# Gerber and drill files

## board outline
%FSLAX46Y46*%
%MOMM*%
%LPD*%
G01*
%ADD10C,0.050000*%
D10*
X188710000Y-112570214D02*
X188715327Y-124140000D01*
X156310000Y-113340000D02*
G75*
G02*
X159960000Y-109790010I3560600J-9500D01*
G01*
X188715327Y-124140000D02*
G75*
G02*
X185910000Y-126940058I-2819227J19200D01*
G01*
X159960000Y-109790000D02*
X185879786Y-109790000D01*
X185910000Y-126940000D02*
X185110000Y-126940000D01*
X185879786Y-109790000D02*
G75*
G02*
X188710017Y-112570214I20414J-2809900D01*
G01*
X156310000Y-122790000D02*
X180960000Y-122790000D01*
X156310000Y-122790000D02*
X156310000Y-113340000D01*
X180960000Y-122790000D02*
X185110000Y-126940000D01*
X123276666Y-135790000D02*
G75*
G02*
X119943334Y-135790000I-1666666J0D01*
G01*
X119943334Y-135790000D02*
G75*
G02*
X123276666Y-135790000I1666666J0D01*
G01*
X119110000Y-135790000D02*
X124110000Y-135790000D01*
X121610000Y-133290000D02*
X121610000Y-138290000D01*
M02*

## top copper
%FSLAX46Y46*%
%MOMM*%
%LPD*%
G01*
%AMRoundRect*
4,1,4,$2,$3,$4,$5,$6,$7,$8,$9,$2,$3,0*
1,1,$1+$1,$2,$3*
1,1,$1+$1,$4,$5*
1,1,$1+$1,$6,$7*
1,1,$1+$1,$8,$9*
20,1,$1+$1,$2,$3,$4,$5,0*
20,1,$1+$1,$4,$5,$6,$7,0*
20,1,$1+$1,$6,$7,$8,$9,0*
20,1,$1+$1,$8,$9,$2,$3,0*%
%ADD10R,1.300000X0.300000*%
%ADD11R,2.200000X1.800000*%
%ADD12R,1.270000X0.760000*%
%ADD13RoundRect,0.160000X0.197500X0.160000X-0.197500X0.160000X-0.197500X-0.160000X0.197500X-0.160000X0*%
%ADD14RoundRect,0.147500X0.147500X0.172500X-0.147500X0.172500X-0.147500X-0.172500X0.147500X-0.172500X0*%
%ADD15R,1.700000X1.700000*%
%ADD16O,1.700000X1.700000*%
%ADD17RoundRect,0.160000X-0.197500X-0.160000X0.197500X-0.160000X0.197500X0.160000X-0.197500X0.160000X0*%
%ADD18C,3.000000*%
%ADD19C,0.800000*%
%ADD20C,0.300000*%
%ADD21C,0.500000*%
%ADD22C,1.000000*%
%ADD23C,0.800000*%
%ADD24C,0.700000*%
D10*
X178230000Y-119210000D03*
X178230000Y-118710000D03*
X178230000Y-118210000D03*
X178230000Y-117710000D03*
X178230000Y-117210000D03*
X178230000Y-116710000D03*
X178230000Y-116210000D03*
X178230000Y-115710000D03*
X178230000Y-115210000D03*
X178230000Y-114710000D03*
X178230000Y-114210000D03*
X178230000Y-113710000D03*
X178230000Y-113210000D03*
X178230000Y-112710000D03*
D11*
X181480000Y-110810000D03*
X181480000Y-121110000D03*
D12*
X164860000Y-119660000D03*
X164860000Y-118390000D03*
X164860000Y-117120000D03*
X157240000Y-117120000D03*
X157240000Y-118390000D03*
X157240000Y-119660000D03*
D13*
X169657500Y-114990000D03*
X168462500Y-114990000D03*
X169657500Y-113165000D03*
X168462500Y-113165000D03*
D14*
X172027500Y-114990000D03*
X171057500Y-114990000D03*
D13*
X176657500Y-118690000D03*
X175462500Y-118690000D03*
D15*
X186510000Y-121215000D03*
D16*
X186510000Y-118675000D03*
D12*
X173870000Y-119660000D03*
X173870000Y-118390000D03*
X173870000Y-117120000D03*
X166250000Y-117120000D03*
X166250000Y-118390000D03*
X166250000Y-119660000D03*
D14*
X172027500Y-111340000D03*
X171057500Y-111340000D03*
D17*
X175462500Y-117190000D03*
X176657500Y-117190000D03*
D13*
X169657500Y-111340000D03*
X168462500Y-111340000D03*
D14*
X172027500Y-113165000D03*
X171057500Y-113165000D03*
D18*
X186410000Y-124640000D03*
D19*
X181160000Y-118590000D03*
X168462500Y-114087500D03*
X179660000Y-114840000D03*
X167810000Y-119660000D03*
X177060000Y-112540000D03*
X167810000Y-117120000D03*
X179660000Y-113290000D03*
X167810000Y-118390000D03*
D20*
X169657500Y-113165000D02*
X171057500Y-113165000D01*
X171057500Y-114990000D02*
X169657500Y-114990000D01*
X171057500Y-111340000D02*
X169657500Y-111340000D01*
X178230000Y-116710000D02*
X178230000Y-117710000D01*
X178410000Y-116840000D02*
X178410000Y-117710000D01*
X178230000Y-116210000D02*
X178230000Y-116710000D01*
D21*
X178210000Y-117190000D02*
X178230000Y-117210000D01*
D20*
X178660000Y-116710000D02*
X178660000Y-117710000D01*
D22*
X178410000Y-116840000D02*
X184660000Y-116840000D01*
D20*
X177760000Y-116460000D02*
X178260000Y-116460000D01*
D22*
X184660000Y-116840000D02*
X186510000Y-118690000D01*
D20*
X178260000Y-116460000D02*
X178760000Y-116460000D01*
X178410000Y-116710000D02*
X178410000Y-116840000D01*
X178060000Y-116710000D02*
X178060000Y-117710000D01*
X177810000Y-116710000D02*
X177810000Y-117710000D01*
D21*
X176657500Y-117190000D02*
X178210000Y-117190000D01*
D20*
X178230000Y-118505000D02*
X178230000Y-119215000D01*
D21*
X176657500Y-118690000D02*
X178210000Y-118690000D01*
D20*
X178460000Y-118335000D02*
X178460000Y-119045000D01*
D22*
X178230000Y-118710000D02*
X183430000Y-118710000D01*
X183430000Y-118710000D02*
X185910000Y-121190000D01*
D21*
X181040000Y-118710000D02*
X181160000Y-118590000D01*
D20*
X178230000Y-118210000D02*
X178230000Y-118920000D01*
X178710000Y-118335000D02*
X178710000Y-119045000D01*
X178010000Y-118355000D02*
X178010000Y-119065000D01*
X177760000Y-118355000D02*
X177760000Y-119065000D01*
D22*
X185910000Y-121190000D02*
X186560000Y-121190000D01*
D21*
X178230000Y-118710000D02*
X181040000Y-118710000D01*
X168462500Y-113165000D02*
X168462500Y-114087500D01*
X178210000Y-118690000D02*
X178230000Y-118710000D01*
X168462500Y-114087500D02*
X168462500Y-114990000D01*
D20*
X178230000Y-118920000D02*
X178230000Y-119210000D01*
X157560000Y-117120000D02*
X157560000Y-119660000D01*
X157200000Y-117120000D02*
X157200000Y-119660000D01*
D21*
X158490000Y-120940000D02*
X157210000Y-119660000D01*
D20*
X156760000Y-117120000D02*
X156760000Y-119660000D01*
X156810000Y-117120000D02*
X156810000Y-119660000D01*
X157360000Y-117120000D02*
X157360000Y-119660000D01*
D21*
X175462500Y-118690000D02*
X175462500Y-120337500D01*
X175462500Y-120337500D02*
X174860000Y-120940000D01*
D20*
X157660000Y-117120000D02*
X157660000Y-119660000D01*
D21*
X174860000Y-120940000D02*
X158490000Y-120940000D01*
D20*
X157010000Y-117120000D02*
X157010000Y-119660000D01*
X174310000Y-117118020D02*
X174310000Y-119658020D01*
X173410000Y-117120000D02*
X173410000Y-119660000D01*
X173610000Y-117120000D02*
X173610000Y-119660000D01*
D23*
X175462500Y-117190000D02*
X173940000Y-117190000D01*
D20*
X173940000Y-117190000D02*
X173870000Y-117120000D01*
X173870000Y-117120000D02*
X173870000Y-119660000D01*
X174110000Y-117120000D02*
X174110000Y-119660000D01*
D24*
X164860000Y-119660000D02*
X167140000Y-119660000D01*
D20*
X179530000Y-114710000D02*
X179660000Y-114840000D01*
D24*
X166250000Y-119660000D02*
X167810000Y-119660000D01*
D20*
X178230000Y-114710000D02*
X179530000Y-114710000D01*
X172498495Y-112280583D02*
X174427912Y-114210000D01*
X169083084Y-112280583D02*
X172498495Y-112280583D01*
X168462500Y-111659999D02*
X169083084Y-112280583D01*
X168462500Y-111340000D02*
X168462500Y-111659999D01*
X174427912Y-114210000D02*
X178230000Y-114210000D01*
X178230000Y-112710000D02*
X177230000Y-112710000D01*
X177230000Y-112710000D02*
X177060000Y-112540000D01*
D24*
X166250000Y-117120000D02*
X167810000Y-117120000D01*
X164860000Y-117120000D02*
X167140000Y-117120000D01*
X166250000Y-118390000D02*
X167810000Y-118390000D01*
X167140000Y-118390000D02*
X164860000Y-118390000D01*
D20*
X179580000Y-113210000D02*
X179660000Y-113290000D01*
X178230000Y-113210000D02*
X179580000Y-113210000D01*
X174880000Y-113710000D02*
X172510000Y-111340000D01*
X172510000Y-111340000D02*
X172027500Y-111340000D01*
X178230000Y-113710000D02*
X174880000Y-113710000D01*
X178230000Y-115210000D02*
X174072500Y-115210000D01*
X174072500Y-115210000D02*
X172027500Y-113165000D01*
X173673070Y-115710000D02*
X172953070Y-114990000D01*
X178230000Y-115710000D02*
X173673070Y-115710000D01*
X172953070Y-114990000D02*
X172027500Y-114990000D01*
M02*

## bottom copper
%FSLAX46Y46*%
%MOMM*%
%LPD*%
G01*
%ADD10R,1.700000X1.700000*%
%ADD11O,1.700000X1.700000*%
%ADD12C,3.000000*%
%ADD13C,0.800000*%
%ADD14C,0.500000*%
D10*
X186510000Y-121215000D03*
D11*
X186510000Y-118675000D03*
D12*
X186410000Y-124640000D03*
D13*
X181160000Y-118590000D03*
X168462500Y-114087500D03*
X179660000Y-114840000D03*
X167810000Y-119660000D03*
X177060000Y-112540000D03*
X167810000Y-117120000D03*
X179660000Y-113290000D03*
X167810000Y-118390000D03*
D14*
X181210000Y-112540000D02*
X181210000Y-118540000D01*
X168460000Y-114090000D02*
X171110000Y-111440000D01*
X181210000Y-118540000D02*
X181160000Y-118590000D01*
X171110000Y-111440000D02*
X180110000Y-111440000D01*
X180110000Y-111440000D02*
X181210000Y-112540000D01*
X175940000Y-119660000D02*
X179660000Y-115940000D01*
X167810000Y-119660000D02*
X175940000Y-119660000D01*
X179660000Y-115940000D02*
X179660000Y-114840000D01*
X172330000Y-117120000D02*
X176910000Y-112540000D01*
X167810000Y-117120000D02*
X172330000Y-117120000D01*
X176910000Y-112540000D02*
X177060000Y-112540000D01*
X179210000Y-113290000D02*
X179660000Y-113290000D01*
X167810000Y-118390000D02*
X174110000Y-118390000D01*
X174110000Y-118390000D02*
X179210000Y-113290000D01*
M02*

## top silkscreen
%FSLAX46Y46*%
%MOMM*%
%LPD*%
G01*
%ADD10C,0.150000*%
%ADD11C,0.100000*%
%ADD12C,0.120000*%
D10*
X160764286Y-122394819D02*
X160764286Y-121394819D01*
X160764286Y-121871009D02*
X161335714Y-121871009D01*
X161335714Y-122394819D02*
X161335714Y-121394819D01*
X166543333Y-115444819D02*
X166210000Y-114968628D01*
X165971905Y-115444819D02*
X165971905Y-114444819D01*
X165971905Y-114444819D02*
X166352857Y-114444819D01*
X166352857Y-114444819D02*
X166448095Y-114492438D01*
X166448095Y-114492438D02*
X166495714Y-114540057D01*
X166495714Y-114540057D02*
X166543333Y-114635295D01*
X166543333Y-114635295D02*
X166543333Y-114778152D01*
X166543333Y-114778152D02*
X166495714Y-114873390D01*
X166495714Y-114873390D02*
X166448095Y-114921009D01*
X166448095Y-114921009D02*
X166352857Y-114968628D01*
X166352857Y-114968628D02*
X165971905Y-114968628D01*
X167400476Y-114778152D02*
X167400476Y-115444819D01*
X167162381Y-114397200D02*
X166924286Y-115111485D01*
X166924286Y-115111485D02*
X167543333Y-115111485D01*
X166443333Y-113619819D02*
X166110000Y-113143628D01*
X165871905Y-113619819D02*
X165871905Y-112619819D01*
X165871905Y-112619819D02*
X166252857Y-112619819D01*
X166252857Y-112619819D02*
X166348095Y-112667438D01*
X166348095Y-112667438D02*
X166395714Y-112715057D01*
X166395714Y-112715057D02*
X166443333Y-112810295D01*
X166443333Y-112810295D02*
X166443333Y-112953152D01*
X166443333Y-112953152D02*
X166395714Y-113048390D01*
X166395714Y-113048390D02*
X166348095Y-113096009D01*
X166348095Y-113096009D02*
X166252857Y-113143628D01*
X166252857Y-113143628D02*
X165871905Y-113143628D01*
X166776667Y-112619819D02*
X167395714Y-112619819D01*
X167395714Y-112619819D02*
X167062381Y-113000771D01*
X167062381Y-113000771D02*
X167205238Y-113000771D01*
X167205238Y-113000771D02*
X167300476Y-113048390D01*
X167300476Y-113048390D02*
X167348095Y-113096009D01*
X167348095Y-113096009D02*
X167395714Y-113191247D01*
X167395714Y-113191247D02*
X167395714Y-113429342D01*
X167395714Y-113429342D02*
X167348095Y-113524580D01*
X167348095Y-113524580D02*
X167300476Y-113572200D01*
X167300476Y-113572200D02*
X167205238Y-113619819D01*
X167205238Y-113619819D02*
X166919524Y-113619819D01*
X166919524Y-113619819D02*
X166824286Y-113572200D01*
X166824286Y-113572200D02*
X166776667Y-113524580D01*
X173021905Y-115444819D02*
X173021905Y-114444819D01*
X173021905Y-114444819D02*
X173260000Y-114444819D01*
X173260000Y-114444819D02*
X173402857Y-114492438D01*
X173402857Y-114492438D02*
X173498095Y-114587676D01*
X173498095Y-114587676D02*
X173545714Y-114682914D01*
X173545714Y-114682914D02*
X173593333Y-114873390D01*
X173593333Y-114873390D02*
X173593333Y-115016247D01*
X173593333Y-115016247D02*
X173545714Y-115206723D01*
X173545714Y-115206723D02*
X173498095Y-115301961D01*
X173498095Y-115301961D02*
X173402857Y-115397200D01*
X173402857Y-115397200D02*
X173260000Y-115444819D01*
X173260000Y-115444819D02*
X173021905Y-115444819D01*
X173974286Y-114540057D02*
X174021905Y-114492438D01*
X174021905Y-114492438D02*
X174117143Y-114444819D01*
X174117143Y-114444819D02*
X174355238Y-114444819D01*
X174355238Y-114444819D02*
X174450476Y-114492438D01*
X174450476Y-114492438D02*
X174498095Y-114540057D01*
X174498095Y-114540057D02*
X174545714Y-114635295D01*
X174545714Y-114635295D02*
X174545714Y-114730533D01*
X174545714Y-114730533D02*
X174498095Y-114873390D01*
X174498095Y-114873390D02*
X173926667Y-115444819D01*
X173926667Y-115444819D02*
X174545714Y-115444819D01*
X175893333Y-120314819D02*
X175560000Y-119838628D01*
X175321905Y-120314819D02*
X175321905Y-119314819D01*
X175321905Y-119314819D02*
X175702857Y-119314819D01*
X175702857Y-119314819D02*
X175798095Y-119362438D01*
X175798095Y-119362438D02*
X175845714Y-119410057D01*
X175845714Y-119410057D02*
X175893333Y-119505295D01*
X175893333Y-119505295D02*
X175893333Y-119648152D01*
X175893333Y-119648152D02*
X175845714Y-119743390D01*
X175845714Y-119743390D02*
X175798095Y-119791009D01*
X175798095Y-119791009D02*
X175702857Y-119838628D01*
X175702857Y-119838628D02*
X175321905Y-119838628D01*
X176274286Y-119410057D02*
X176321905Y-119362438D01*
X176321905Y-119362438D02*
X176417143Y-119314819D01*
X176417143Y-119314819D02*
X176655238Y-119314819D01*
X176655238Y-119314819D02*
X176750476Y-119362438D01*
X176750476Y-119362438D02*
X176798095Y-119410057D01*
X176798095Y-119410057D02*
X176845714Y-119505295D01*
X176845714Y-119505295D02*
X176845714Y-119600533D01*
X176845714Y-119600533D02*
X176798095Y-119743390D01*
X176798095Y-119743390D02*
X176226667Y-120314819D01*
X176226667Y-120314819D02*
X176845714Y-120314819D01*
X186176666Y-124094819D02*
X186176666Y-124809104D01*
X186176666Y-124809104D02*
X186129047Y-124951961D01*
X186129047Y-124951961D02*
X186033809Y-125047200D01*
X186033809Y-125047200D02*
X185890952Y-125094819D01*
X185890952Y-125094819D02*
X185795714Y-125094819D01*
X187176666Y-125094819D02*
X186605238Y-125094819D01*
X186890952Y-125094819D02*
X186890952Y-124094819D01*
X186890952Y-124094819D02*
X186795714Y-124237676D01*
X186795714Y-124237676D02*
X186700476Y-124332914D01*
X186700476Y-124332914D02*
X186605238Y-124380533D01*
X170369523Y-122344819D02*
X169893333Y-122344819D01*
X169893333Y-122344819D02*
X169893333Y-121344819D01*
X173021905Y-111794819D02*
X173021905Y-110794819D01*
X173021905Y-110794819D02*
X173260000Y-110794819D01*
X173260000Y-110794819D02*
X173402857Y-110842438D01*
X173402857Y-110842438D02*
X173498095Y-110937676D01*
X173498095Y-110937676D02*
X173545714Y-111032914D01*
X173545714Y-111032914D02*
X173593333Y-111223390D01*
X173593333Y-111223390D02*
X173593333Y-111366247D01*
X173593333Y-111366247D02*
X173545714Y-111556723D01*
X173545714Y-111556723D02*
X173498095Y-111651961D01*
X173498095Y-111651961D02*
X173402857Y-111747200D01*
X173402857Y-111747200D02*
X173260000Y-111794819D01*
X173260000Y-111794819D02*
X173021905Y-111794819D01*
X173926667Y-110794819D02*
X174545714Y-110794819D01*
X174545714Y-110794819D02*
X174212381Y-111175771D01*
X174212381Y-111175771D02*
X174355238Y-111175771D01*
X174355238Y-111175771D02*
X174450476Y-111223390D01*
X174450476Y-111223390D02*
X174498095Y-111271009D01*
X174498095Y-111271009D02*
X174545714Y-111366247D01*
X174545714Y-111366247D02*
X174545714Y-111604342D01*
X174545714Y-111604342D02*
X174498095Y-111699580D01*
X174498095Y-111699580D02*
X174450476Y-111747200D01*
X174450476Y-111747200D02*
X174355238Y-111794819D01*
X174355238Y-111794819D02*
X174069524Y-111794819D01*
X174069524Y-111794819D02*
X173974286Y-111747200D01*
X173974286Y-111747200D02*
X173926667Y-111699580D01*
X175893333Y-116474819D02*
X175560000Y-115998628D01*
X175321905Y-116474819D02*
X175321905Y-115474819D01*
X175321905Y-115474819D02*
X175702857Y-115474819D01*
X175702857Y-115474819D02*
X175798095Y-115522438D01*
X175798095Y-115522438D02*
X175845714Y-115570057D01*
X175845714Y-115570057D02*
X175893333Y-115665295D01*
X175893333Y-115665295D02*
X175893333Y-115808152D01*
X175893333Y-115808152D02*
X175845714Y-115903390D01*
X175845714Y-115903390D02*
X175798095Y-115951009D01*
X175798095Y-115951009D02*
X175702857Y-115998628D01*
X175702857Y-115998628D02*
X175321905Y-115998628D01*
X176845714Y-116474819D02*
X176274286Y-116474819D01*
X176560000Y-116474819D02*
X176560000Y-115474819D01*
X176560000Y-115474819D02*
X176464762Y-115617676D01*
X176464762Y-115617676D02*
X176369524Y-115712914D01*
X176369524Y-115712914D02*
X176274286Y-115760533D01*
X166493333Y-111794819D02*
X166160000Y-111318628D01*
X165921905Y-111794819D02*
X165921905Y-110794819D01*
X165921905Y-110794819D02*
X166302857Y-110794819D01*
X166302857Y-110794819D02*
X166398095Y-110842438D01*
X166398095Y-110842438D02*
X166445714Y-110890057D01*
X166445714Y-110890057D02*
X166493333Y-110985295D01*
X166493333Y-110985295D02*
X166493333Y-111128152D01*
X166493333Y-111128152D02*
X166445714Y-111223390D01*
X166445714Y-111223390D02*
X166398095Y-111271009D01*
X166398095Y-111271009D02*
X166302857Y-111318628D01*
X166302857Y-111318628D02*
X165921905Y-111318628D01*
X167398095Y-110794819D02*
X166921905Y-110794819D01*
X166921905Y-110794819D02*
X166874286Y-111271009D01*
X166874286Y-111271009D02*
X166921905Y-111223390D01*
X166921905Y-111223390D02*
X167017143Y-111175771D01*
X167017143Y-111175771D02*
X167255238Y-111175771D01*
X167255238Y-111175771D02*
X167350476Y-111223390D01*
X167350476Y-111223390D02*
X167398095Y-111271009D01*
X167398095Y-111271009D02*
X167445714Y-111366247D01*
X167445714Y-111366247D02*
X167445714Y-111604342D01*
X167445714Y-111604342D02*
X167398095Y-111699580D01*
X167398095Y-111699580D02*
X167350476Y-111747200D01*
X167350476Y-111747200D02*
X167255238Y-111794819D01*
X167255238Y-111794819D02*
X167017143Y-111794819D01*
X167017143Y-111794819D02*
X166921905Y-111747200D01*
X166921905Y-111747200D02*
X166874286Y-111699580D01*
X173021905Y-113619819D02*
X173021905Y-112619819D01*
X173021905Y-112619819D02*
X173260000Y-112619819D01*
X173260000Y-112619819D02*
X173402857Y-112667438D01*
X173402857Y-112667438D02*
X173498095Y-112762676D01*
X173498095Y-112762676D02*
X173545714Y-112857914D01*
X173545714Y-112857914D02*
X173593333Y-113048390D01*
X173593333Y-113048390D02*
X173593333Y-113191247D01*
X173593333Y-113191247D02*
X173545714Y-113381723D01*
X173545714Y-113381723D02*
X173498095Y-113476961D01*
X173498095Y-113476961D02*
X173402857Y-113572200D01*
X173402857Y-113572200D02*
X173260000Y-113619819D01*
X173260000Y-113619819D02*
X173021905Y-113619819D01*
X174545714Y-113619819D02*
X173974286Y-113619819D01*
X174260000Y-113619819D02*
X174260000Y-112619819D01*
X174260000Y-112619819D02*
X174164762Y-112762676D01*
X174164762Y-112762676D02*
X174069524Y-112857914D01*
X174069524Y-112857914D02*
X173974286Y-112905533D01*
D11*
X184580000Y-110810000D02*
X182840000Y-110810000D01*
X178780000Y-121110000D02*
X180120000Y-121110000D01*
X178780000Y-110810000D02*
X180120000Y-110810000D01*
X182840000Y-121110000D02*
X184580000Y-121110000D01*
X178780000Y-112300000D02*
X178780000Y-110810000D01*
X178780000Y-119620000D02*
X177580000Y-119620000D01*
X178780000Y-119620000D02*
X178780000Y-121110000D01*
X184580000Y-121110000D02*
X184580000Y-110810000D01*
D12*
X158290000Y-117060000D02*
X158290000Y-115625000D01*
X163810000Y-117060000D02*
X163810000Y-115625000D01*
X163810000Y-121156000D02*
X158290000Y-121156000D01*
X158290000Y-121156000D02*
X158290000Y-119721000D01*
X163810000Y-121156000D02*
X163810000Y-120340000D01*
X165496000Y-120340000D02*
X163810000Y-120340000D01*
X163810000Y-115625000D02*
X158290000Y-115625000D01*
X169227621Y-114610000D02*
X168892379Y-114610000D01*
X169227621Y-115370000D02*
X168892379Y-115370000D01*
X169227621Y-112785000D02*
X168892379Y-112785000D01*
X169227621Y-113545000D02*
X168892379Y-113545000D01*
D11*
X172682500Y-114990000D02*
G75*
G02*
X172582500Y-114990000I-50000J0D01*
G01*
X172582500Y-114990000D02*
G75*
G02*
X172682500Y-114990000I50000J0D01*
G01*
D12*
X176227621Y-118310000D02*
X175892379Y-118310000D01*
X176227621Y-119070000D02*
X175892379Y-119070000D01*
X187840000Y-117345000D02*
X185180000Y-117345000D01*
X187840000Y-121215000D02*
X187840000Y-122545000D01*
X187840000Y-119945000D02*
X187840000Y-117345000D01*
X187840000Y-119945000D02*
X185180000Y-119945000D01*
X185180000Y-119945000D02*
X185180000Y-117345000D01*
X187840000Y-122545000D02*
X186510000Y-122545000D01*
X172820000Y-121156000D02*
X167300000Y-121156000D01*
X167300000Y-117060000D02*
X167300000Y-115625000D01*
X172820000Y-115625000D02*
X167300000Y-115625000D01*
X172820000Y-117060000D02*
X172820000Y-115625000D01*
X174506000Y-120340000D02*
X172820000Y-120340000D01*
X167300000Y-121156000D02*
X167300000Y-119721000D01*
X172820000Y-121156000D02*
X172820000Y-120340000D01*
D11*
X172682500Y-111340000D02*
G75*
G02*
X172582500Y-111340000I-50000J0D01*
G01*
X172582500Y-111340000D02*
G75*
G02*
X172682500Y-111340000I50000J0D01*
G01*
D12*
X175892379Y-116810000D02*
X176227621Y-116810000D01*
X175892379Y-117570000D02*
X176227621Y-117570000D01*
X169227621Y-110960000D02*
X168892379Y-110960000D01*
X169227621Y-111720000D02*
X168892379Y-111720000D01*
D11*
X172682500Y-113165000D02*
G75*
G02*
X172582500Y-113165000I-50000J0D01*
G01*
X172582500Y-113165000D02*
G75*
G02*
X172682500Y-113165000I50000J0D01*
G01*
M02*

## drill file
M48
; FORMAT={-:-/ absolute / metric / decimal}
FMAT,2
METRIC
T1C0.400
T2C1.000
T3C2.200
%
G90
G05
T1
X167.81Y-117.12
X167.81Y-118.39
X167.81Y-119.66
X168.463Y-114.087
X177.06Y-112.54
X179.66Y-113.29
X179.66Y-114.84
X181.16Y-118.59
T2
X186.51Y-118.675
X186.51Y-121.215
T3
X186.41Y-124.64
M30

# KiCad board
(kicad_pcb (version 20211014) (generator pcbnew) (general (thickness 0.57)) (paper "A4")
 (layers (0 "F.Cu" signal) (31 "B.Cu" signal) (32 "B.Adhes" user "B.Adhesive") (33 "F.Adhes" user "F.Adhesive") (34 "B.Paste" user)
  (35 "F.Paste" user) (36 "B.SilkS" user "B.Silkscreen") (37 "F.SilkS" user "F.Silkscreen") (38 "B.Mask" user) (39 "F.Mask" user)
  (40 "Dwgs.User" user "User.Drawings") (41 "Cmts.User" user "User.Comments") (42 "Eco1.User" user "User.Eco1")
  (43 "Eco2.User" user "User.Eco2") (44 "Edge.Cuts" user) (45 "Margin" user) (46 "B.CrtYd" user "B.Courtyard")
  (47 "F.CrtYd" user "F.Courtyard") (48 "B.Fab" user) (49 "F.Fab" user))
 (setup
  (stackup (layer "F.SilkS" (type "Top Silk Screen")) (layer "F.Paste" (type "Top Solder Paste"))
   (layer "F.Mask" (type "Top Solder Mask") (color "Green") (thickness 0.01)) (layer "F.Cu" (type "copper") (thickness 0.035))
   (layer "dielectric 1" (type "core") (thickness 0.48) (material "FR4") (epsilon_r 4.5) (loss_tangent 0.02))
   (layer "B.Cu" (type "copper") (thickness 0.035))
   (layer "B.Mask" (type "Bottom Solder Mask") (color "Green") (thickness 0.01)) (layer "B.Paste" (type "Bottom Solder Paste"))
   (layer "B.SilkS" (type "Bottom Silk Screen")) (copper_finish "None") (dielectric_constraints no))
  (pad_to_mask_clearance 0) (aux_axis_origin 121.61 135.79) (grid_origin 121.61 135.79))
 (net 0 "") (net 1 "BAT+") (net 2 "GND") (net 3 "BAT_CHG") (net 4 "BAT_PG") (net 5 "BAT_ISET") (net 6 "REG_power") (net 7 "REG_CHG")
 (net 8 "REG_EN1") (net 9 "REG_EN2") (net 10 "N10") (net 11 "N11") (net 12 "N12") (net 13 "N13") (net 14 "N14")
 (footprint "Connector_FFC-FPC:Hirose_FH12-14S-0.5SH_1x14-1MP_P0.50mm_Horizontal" (layer "F.Cu") (at 180.08 115.96 90)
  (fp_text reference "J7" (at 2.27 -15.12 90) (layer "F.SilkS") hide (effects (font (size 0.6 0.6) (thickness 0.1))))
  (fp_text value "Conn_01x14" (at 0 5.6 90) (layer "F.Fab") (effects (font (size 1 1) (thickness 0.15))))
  (fp_line (start 5.15 4.5) (end 5.15 2.76) (layer "F.SilkS") (width 0.1))
  (fp_line (start -5.15 -1.3) (end -5.15 0.04) (layer "F.SilkS") (width 0.1))
  (fp_line (start 5.15 -1.3) (end 5.15 0.04) (layer "F.SilkS") (width 0.1))
  (fp_line (start -5.15 2.76) (end -5.15 4.5) (layer "F.SilkS") (width 0.1))
  (fp_line (start 3.66 -1.3) (end 5.15 -1.3) (layer "F.SilkS") (width 0.1))
  (fp_line (start -3.66 -1.3) (end -3.66 -2.5) (layer "F.SilkS") (width 0.1))
  (fp_line (start -3.66 -1.3) (end -5.15 -1.3) (layer "F.SilkS") (width 0.1))
  (fp_line (start -5.15 4.5) (end 5.15 4.5) (layer "F.SilkS") (width 0.1))
  (pad "1" smd rect locked (at -3.25 -1.85 90) (size 0.3 1.3) (layers "F.Cu" "F.Paste" "F.Mask") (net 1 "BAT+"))
  (pad "2" smd rect locked (at -2.75 -1.85 90) (size 0.3 1.3) (layers "F.Cu" "F.Paste" "F.Mask") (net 1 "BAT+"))
  (pad "3" smd rect locked (at -2.25 -1.85 90) (size 0.3 1.3) (layers "F.Cu" "F.Paste" "F.Mask") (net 1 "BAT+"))
  (pad "4" smd rect locked (at -1.75 -1.85 90) (size 0.3 1.3) (layers "F.Cu" "F.Paste" "F.Mask") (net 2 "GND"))
  (pad "5" smd rect locked (at -1.25 -1.85 90) (size 0.3 1.3) (layers "F.Cu" "F.Paste" "F.Mask") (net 2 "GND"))
  (pad "6" smd rect locked (at -0.75 -1.85 90) (size 0.3 1.3) (layers "F.Cu" "F.Paste" "F.Mask") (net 2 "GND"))
  (pad "7" smd rect locked (at -0.25 -1.85 90) (size 0.3 1.3) (layers "F.Cu" "F.Paste" "F.Mask") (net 2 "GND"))
  (pad "8" smd rect locked (at 0.25 -1.85 90) (size 0.3 1.3) (layers "F.Cu" "F.Paste" "F.Mask") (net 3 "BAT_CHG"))
  (pad "9" smd rect locked (at 0.75 -1.85 90) (size 0.3 1.3) (layers "F.Cu" "F.Paste" "F.Mask") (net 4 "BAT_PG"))
  (pad "10" smd rect locked (at 1.25 -1.85 90) (size 0.3 1.3) (layers "F.Cu" "F.Paste" "F.Mask") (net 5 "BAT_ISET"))
  (pad "11" smd rect locked (at 1.75 -1.85 90) (size 0.3 1.3) (layers "F.Cu" "F.Paste" "F.Mask") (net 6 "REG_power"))
  (pad "12" smd rect locked (at 2.25 -1.85 90) (size 0.3 1.3) (layers "F.Cu" "F.Paste" "F.Mask") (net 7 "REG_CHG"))
  (pad "13" smd rect locked (at 2.75 -1.85 90) (size 0.3 1.3) (layers "F.Cu" "F.Paste" "F.Mask") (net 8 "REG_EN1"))
  (pad "14" smd rect locked (at 3.25 -1.85 90) (size 0.3 1.3) (layers "F.Cu" "F.Paste" "F.Mask") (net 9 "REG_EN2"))
  (pad "MP" smd rect locked (at 5.15 1.4 90) (size 1.8 2.2) (layers "F.Cu" "F.Paste" "F.Mask"))
  (pad "MP" smd rect locked (at -5.15 1.4 90) (size 1.8 2.2) (layers "F.Cu" "F.Paste" "F.Mask")))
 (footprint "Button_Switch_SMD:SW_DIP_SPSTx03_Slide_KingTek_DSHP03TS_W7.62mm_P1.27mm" (layer "F.Cu") (at 161.05 118.39 180)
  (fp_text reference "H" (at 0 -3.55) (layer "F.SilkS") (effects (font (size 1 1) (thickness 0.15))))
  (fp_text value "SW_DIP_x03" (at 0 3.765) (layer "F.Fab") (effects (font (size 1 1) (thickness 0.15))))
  (fp_line (start 2.76 1.33) (end 2.76 2.765) (layer "F.SilkS") (width 0.12))
  (fp_line (start -2.76 1.33) (end -2.76 2.765) (layer "F.SilkS") (width 0.12))
  (fp_line (start -2.76 -2.766) (end 2.76 -2.766) (layer "F.SilkS") (width 0.12))
  (fp_line (start 2.76 -2.766) (end 2.76 -1.331) (layer "F.SilkS") (width 0.12))
  (fp_line (start -2.76 -2.766) (end -2.76 -1.95) (layer "F.SilkS") (width 0.12))
  (fp_line (start -4.446 -1.95) (end -2.76 -1.95) (layer "F.SilkS") (width 0.12))
  (fp_line (start -2.76 2.765) (end 2.76 2.765) (layer "F.SilkS") (width 0.12))
  (pad "1" smd rect locked (at -3.81 -1.27 180) (size 1.27 0.76) (layers "F.Cu" "F.Paste" "F.Mask") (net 5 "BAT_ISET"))
  (pad "2" smd rect locked (at -3.81 0 180) (size 1.27 0.76) (layers "F.Cu" "F.Paste" "F.Mask") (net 8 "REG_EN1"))
  (pad "3" smd rect locked (at -3.81 1.27 180) (size 1.27 0.76) (layers "F.Cu" "F.Paste" "F.Mask") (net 9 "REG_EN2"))
  (pad "4" smd rect locked (at 3.81 1.27 180) (size 1.27 0.76) (layers "F.Cu" "F.Paste" "F.Mask") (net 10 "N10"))
  (pad "5" smd rect locked (at 3.81 0 180) (size 1.27 0.76) (layers "F.Cu" "F.Paste" "F.Mask") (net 10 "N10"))
  (pad "6" smd rect locked (at 3.81 -1.27 180) (size 1.27 0.76) (layers "F.Cu" "F.Paste" "F.Mask") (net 10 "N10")))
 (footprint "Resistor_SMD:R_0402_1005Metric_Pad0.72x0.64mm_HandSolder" (layer "F.Cu") (at 169.06 114.99 180)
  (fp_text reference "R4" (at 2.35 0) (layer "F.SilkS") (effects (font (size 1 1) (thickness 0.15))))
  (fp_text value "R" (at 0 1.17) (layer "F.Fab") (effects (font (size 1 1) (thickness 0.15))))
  (fp_line (start -0.167621 0.38) (end 0.167621 0.38) (layer "F.SilkS") (width 0.12))
  (fp_line (start -0.167621 -0.38) (end 0.167621 -0.38) (layer "F.SilkS") (width 0.12))
  (pad "1" smd roundrect locked (at -0.5975 0 180) (size 0.715 0.64) (layers "F.Cu" "F.Paste" "F.Mask") (roundrect_rratio 0.25)
   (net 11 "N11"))
  (pad "2" smd roundrect locked (at 0.5975 0 180) (size 0.715 0.64) (layers "F.Cu" "F.Paste" "F.Mask") (roundrect_rratio 0.25)
   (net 1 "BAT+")))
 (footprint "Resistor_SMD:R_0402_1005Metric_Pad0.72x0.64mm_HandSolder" (layer "F.Cu") (at 169.06 113.165 180)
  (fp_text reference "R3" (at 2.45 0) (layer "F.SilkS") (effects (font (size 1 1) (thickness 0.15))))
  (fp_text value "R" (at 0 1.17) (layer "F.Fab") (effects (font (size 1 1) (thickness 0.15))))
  (fp_line (start -0.167621 0.38) (end 0.167621 0.38) (layer "F.SilkS") (width 0.12))
  (fp_line (start -0.167621 -0.38) (end 0.167621 -0.38) (layer "F.SilkS") (width 0.12))
  (pad "1" smd roundrect locked (at -0.5975 0 180) (size 0.715 0.64) (layers "F.Cu" "F.Paste" "F.Mask") (roundrect_rratio 0.25)
   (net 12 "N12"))
  (pad "2" smd roundrect locked (at 0.5975 0 180) (size 0.715 0.64) (layers "F.Cu" "F.Paste" "F.Mask") (roundrect_rratio 0.25)
   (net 1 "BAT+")))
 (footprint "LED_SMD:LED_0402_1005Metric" (layer "F.Cu") (at 171.5425 114.99 180)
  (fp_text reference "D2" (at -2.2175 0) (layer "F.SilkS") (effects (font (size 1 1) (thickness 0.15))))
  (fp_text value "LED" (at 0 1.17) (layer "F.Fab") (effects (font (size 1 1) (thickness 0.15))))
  (fp_circle (center -1.09 0) (end -1.04 0) (layer "F.SilkS") (width 0.1) (fill none))
  (pad "1" smd roundrect locked (at -0.485 0 180) (size 0.59 0.64) (layers "F.Cu" "F.Paste" "F.Mask") (roundrect_rratio 0.25)
   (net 3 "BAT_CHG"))
  (pad "2" smd roundrect locked (at 0.485 0 180) (size 0.59 0.64) (layers "F.Cu" "F.Paste" "F.Mask") (roundrect_rratio 0.25) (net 11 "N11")))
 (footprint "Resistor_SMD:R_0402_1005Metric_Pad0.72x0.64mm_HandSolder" (layer "F.Cu") (at 176.06 118.69 180)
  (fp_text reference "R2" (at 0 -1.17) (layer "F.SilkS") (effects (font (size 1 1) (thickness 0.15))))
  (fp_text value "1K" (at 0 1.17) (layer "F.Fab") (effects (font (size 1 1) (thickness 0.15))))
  (fp_line (start -0.167621 0.38) (end 0.167621 0.38) (layer "F.SilkS") (width 0.12))
  (fp_line (start -0.167621 -0.38) (end 0.167621 -0.38) (layer "F.SilkS") (width 0.12))
  (pad "1" smd roundrect locked (at -0.5975 0 180) (size 0.715 0.64) (layers "F.Cu" "F.Paste" "F.Mask") (roundrect_rratio 0.25)
   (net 1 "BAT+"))
  (pad "2" smd roundrect locked (at 0.5975 0 180) (size 0.715 0.64) (layers "F.Cu" "F.Paste" "F.Mask") (roundrect_rratio 0.25)
   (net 10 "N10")))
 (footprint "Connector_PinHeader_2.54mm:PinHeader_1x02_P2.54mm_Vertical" (layer "F.Cu") (at 186.51 121.215 180)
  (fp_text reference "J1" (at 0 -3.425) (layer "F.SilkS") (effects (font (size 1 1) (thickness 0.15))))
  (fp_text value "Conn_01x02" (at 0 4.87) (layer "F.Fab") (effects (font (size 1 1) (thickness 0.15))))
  (fp_line (start -1.33 3.87) (end 1.33 3.87) (layer "F.SilkS") (width 0.12))
  (fp_line (start -1.33 0) (end -1.33 -1.33) (layer "F.SilkS") (width 0.12))
  (fp_line (start -1.33 1.27) (end -1.33 3.87) (layer "F.SilkS") (width 0.12))
  (fp_line (start -1.33 1.27) (end 1.33 1.27) (layer "F.SilkS") (width 0.12))
  (fp_line (start 1.33 1.27) (end 1.33 3.87) (layer "F.SilkS") (width 0.12))
  (fp_line (start -1.33 -1.33) (end 0 -1.33) (layer "F.SilkS") (width 0.12))
  (pad "1" thru_hole rect locked (at 0 0 180) (size 1.7 1.7) (drill 1) (layers *.Cu *.Mask) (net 1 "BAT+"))
  (pad "2" thru_hole oval locked (at 0 2.54 180) (size 1.7 1.7) (drill 1) (layers *.Cu *.Mask) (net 2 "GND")))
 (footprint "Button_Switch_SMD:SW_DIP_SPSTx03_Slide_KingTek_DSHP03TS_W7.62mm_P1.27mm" (layer "F.Cu") (at 170.06 118.39 180)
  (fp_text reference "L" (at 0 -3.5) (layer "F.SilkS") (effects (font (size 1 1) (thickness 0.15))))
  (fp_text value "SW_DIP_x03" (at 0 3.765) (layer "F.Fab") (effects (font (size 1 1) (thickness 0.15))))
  (fp_line (start -2.76 -2.766) (end 2.76 -2.766) (layer "F.SilkS") (width 0.12))
  (fp_line (start 2.76 1.33) (end 2.76 2.765) (layer "F.SilkS") (width 0.12))
  (fp_line (start -2.76 2.765) (end 2.76 2.765) (layer "F.SilkS") (width 0.12))
  (fp_line (start -2.76 1.33) (end -2.76 2.765) (layer "F.SilkS") (width 0.12))
  (fp_line (start -4.446 -1.95) (end -2.76 -1.95) (layer "F.SilkS") (width 0.12))
  (fp_line (start 2.76 -2.766) (end 2.76 -1.331) (layer "F.SilkS") (width 0.12))
  (fp_line (start -2.76 -2.766) (end -2.76 -1.95) (layer "F.SilkS") (width 0.12))
  (pad "1" smd rect locked (at -3.81 -1.27 180) (size 1.27 0.76) (layers "F.Cu" "F.Paste" "F.Mask") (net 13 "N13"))
  (pad "2" smd rect locked (at -3.81 0 180) (size 1.27 0.76) (layers "F.Cu" "F.Paste" "F.Mask") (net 13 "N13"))
  (pad "3" smd rect locked (at -3.81 1.27 180) (size 1.27 0.76) (layers "F.Cu" "F.Paste" "F.Mask") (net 13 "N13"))
  (pad "4" smd rect locked (at 3.81 1.27 180) (size 1.27 0.76) (layers "F.Cu" "F.Paste" "F.Mask") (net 9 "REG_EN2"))
  (pad "5" smd rect locked (at 3.81 0 180) (size 1.27 0.76) (layers "F.Cu" "F.Paste" "F.Mask") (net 8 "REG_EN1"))
  (pad "6" smd rect locked (at 3.81 -1.27 180) (size 1.27 0.76) (layers "F.Cu" "F.Paste" "F.Mask") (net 5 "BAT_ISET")))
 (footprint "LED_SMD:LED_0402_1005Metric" (layer "F.Cu") (at 171.5425 111.34 180)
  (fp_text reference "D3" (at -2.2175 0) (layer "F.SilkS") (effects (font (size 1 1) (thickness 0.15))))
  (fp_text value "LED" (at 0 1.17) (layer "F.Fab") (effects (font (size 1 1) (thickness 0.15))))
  (fp_circle (center -1.09 0) (end -1.04 0) (layer "F.SilkS") (width 0.1) (fill none))
  (pad "1" smd roundrect locked (at -0.485 0 180) (size 0.59 0.64) (layers "F.Cu" "F.Paste" "F.Mask") (roundrect_rratio 0.25)
   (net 7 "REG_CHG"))
  (pad "2" smd roundrect locked (at 0.485 0 180) (size 0.59 0.64) (layers "F.Cu" "F.Paste" "F.Mask") (roundrect_rratio 0.25) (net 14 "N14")))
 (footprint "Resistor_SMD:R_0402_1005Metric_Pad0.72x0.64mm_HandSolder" (layer "F.Cu") (at 176.06 117.19)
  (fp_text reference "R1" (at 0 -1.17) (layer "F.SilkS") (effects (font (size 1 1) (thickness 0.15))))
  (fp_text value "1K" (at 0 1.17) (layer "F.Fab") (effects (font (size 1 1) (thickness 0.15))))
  (fp_line (start -0.167621 -0.38) (end 0.167621 -0.38) (layer "F.SilkS") (width 0.12))
  (fp_line (start -0.167621 0.38) (end 0.167621 0.38) (layer "F.SilkS") (width 0.12))
  (pad "1" smd roundrect locked (at -0.5975 0) (size 0.715 0.64) (layers "F.Cu" "F.Paste" "F.Mask") (roundrect_rratio 0.25) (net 13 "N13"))
  (pad "2" smd roundrect locked (at 0.5975 0) (size 0.715 0.64) (layers "F.Cu" "F.Paste" "F.Mask") (roundrect_rratio 0.25) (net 2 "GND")))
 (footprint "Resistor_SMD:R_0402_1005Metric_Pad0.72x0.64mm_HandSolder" (layer "F.Cu") (at 169.06 111.34 180)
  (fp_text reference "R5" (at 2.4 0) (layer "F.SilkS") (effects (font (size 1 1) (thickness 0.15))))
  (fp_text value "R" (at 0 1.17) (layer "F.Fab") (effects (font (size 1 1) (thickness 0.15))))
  (fp_line (start -0.167621 0.38) (end 0.167621 0.38) (layer "F.SilkS") (width 0.12))
  (fp_line (start -0.167621 -0.38) (end 0.167621 -0.38) (layer "F.SilkS") (width 0.12))
  (pad "1" smd roundrect locked (at -0.5975 0 180) (size 0.715 0.64) (layers "F.Cu" "F.Paste" "F.Mask") (roundrect_rratio 0.25)
   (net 14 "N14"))
  (pad "2" smd roundrect locked (at 0.5975 0 180) (size 0.715 0.64) (layers "F.Cu" "F.Paste" "F.Mask") (roundrect_rratio 0.25)
   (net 6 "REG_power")))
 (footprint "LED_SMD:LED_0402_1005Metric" (layer "F.Cu") (at 171.5425 113.165 180)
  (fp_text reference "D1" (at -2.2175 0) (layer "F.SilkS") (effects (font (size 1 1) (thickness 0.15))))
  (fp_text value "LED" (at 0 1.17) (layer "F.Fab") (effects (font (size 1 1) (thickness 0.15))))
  (fp_circle (center -1.09 0) (end -1.04 0) (layer "F.SilkS") (width 0.1) (fill none))
  (pad "1" smd roundrect locked (at -0.485 0 180) (size 0.59 0.64) (layers "F.Cu" "F.Paste" "F.Mask") (roundrect_rratio 0.25)
   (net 4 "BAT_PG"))
  (pad "2" smd roundrect locked (at 0.485 0 180) (size 0.59 0.64) (layers "F.Cu" "F.Paste" "F.Mask") (roundrect_rratio 0.25) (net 12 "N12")))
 (gr_line (start 188.71 112.570214) (end 188.715327 124.14) (layer "Edge.Cuts") (width 0.05))
 (gr_arc (start 156.31 113.34) (mid 157.38808 110.79704) (end 159.96 109.79) (layer "Edge.Cuts") (width 0.05))
 (gr_arc (start 188.715327 124.14) (mid 187.887752 126.116182) (end 185.91 126.94) (layer "Edge.Cuts") (width 0.05))
 (gr_line (start 159.96 109.79) (end 185.879786 109.79) (layer "Edge.Cuts") (width 0.05))
 (gr_line (start 185.91 126.94) (end 185.11 126.94) (layer "Edge.Cuts") (width 0.05))
 (gr_arc (start 185.879786 109.79) (mid 187.869341 110.595327) (end 188.71 112.570214) (layer "Edge.Cuts") (width 0.05))
 (gr_line (start 156.31 122.79) (end 180.96 122.79) (layer "Edge.Cuts") (width 0.05))
 (gr_line (start 156.31 122.79) (end 156.31 113.34) (layer "Edge.Cuts") (width 0.05))
 (gr_line (start 180.96 122.79) (end 185.11 126.94) (layer "Edge.Cuts") (width 0.05))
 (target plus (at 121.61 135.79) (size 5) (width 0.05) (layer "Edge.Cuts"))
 (via (at 186.41 124.64) (size 3) (drill 2.2) (layers "F.Cu" "B.Cu") (free) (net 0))
 (segment (start 169.6575 113.165) (end 171.0575 113.165) (width 0.3) (layer "F.Cu") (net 12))
 (segment (start 171.0575 114.99) (end 169.6575 114.99) (width 0.3) (layer "F.Cu") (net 11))
 (segment (start 171.0575 111.34) (end 169.6575 111.34) (width 0.3) (layer "F.Cu") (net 14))
 (segment (start 178.23 116.71) (end 178.23 117.71) (width 0.3) (layer "F.Cu") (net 2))
 (segment (start 178.41 116.84) (end 178.41 117.71) (width 0.3) (layer "F.Cu") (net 2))
 (segment (start 178.23 116.21) (end 178.23 116.71) (width 0.3) (layer "F.Cu") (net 2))
 (segment (start 178.21 117.19) (end 178.23 117.21) (width 0.5) (layer "F.Cu") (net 2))
 (segment (start 178.66 116.71) (end 178.66 117.71) (width 0.3) (layer "F.Cu") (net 2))
 (segment (start 178.41 116.84) (end 184.66 116.84) (width 1) (layer "F.Cu") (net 2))
 (segment (start 177.76 116.46) (end 178.26 116.46) (width 0.3) (layer "F.Cu") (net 2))
 (segment (start 184.66 116.84) (end 186.51 118.69) (width 1) (layer "F.Cu") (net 2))
 (segment (start 178.26 116.46) (end 178.76 116.46) (width 0.3) (layer "F.Cu") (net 2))
 (segment (start 178.41 116.71) (end 178.41 116.84) (width 0.3) (layer "F.Cu") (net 2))
 (segment (start 178.06 116.71) (end 178.06 117.71) (width 0.3) (layer "F.Cu") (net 2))
 (segment (start 177.81 116.71) (end 177.81 117.71) (width 0.3) (layer "F.Cu") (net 2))
 (segment (start 176.6575 117.19) (end 178.21 117.19) (width 0.5) (layer "F.Cu") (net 2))
 (segment (start 178.23 118.505) (end 178.23 119.215) (width 0.3) (layer "F.Cu") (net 1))
 (segment (start 176.6575 118.69) (end 178.21 118.69) (width 0.5) (layer "F.Cu") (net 1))
 (segment (start 178.46 118.335) (end 178.46 119.045) (width 0.3) (layer "F.Cu") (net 1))
 (segment (start 178.23 118.71) (end 183.43 118.71) (width 1) (layer "F.Cu") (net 1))
 (segment (start 183.43 118.71) (end 185.91 121.19) (width 1) (layer "F.Cu") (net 1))
 (segment (start 181.04 118.71) (end 181.16 118.59) (width 0.5) (layer "F.Cu") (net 1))
 (segment (start 178.23 118.21) (end 178.23 118.92) (width 0.3) (layer "F.Cu") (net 1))
 (segment (start 178.71 118.335) (end 178.71 119.045) (width 0.3) (layer "F.Cu") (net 1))
 (segment (start 178.01 118.355) (end 178.01 119.065) (width 0.3) (layer "F.Cu") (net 1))
 (segment (start 177.76 118.355) (end 177.76 119.065) (width 0.3) (layer "F.Cu") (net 1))
 (segment (start 185.91 121.19) (end 186.56 121.19) (width 1) (layer "F.Cu") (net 1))
 (segment (start 178.23 118.71) (end 181.04 118.71) (width 0.5) (layer "F.Cu") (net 1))
 (segment (start 168.4625 113.165) (end 168.4625 114.0875) (width 0.5) (layer "F.Cu") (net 1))
 (segment (start 178.21 118.69) (end 178.23 118.71) (width 0.5) (layer "F.Cu") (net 1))
 (segment (start 168.4625 114.0875) (end 168.4625 114.99) (width 0.5) (layer "F.Cu") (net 1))
 (segment (start 178.23 118.92) (end 178.23 119.21) (width 0.3) (layer "F.Cu") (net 1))
 (via (at 181.16 118.59) (size 0.8) (drill 0.4) (layers "F.Cu" "B.Cu") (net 1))
 (via (at 168.4625 114.0875) (size 0.8) (drill 0.4) (layers "F.Cu" "B.Cu") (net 1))
 (segment (start 181.21 112.54) (end 181.21 118.54) (width 0.5) (layer "B.Cu") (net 1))
 (segment (start 168.46 114.09) (end 171.11 111.44) (width 0.5) (layer "B.Cu") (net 1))
 (segment (start 181.21 118.54) (end 181.16 118.59) (width 0.5) (layer "B.Cu") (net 1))
 (segment (start 171.11 111.44) (end 180.11 111.44) (width 0.5) (layer "B.Cu") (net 1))
 (segment (start 180.11 111.44) (end 181.21 112.54) (width 0.5) (layer "B.Cu") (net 1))
 (segment (start 157.56 117.12) (end 157.56 119.66) (width 0.3) (layer "F.Cu") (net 10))
 (segment (start 157.2 117.12) (end 157.2 119.66) (width 0.3) (layer "F.Cu") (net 10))
 (segment (start 158.49 120.94) (end 157.21 119.66) (width 0.5) (layer "F.Cu") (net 10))
 (segment (start 156.76 117.12) (end 156.76 119.66) (width 0.3) (layer "F.Cu") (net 10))
 (segment (start 156.81 117.12) (end 156.81 119.66) (width 0.3) (layer "F.Cu") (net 10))
 (segment (start 157.36 117.12) (end 157.36 119.66) (width 0.3) (layer "F.Cu") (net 10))
 (segment (start 175.4625 118.69) (end 175.4625 120.3375) (width 0.5) (layer "F.Cu") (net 10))
 (segment (start 175.4625 120.3375) (end 174.86 120.94) (width 0.5) (layer "F.Cu") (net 10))
 (segment (start 157.66 117.12) (end 157.66 119.66) (width 0.3) (layer "F.Cu") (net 10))
 (segment (start 174.86 120.94) (end 158.49 120.94) (width 0.5) (layer "F.Cu") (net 10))
 (segment (start 157.01 117.12) (end 157.01 119.66) (width 0.3) (layer "F.Cu") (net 10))
 (segment (start 174.31 117.11802) (end 174.31 119.65802) (width 0.3) (layer "F.Cu") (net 13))
 (segment (start 173.41 117.12) (end 173.41 119.66) (width 0.3) (layer "F.Cu") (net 13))
 (segment (start 173.61 117.12) (end 173.61 119.66) (width 0.3) (layer "F.Cu") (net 13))
 (segment (start 175.4625 117.19) (end 173.94 117.19) (width 0.8) (layer "F.Cu") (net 13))
 (segment (start 173.94 117.19) (end 173.87 117.12) (width 0.3) (layer "F.Cu") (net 13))
 (segment (start 173.87 117.12) (end 173.87 119.66) (width 0.3) (layer "F.Cu") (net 13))
 (segment (start 174.11 117.12) (end 174.11 119.66) (width 0.3) (layer "F.Cu") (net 13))
 (segment (start 164.86 119.66) (end 167.14 119.66) (width 0.7) (layer "F.Cu") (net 5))
 (segment (start 179.53 114.71) (end 179.66 114.84) (width 0.3) (layer "F.Cu") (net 5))
 (segment (start 166.25 119.66) (end 167.81 119.66) (width 0.7) (layer "F.Cu") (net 5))
 (segment (start 178.23 114.71) (end 179.53 114.71) (width 0.3) (layer "F.Cu") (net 5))
 (via (at 179.66 114.84) (size 0.8) (drill 0.4) (layers "F.Cu" "B.Cu") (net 5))
 (via (at 167.81 119.66) (size 0.8) (drill 0.4) (layers "F.Cu" "B.Cu") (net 5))
 (segment (start 175.94 119.66) (end 179.66 115.94) (width 0.5) (layer "B.Cu") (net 5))
 (segment (start 167.81 119.66) (end 175.94 119.66) (width 0.5) (layer "B.Cu") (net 5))
 (segment (start 179.66 115.94) (end 179.66 114.84) (width 0.5) (layer "B.Cu") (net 5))
 (segment (start 172.498495 112.280583) (end 174.427912 114.21) (width 0.3) (layer "F.Cu") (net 6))
 (segment (start 169.083084 112.280583) (end 172.498495 112.280583) (width 0.3) (layer "F.Cu") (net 6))
 (segment (start 168.4625 111.659999) (end 169.083084 112.280583) (width 0.3) (layer "F.Cu") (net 6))
 (segment (start 168.4625 111.34) (end 168.4625 111.659999) (width 0.3) (layer "F.Cu") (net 6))
 (segment (start 174.427912 114.21) (end 178.23 114.21) (width 0.3) (layer "F.Cu") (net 6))
 (segment (start 178.23 112.71) (end 177.23 112.71) (width 0.3) (layer "F.Cu") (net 9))
 (segment (start 177.23 112.71) (end 177.06 112.54) (width 0.3) (layer "F.Cu") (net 9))
 (segment (start 166.25 117.12) (end 167.81 117.12) (width 0.7) (layer "F.Cu") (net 9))
 (segment (start 164.86 117.12) (end 167.14 117.12) (width 0.7) (layer "F.Cu") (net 9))
 (via (at 177.06 112.54) (size 0.8) (drill 0.4) (layers "F.Cu" "B.Cu") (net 9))
 (via (at 167.81 117.12) (size 0.8) (drill 0.4) (layers "F.Cu" "B.Cu") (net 9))
 (segment (start 172.33 117.12) (end 176.91 112.54) (width 0.5) (layer "B.Cu") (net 9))
 (segment (start 167.81 117.12) (end 172.33 117.12) (width 0.5) (layer "B.Cu") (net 9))
 (segment (start 176.91 112.54) (end 177.06 112.54) (width 0.5) (layer "B.Cu") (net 9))
 (segment (start 166.25 118.39) (end 167.81 118.39) (width 0.7) (layer "F.Cu") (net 8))
 (segment (start 167.14 118.39) (end 164.86 118.39) (width 0.7) (layer "F.Cu") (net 8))
 (segment (start 179.58 113.21) (end 179.66 113.29) (width 0.3) (layer "F.Cu") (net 8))
 (segment (start 178.23 113.21) (end 179.58 113.21) (width 0.3) (layer "F.Cu") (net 8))
 (via (at 179.66 113.29) (size 0.8) (drill 0.4) (layers "F.Cu" "B.Cu") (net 8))
 (via (at 167.81 118.39) (size 0.8) (drill 0.4) (layers "F.Cu" "B.Cu") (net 8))
 (segment (start 179.21 113.29) (end 179.66 113.29) (width 0.5) (layer "B.Cu") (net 8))
 (segment (start 167.81 118.39) (end 174.11 118.39) (width 0.5) (layer "B.Cu") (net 8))
 (segment (start 174.11 118.39) (end 179.21 113.29) (width 0.5) (layer "B.Cu") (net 8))
 (segment (start 174.88 113.71) (end 172.51 111.34) (width 0.3) (layer "F.Cu") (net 7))
 (segment (start 172.51 111.34) (end 172.0275 111.34) (width 0.3) (layer "F.Cu") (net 7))
 (segment (start 178.23 113.71) (end 174.88 113.71) (width 0.3) (layer "F.Cu") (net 7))
 (segment (start 178.23 115.21) (end 174.0725 115.21) (width 0.3) (layer "F.Cu") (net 4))
 (segment (start 174.0725 115.21) (end 172.0275 113.165) (width 0.3) (layer "F.Cu") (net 4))
 (segment (start 173.67307 115.71) (end 172.95307 114.99) (width 0.3) (layer "F.Cu") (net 3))
 (segment (start 178.23 115.71) (end 173.67307 115.71) (width 0.3) (layer "F.Cu") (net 3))
 (segment (start 172.95307 114.99) (end 172.0275 114.99) (width 0.3) (layer "F.Cu") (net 3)))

